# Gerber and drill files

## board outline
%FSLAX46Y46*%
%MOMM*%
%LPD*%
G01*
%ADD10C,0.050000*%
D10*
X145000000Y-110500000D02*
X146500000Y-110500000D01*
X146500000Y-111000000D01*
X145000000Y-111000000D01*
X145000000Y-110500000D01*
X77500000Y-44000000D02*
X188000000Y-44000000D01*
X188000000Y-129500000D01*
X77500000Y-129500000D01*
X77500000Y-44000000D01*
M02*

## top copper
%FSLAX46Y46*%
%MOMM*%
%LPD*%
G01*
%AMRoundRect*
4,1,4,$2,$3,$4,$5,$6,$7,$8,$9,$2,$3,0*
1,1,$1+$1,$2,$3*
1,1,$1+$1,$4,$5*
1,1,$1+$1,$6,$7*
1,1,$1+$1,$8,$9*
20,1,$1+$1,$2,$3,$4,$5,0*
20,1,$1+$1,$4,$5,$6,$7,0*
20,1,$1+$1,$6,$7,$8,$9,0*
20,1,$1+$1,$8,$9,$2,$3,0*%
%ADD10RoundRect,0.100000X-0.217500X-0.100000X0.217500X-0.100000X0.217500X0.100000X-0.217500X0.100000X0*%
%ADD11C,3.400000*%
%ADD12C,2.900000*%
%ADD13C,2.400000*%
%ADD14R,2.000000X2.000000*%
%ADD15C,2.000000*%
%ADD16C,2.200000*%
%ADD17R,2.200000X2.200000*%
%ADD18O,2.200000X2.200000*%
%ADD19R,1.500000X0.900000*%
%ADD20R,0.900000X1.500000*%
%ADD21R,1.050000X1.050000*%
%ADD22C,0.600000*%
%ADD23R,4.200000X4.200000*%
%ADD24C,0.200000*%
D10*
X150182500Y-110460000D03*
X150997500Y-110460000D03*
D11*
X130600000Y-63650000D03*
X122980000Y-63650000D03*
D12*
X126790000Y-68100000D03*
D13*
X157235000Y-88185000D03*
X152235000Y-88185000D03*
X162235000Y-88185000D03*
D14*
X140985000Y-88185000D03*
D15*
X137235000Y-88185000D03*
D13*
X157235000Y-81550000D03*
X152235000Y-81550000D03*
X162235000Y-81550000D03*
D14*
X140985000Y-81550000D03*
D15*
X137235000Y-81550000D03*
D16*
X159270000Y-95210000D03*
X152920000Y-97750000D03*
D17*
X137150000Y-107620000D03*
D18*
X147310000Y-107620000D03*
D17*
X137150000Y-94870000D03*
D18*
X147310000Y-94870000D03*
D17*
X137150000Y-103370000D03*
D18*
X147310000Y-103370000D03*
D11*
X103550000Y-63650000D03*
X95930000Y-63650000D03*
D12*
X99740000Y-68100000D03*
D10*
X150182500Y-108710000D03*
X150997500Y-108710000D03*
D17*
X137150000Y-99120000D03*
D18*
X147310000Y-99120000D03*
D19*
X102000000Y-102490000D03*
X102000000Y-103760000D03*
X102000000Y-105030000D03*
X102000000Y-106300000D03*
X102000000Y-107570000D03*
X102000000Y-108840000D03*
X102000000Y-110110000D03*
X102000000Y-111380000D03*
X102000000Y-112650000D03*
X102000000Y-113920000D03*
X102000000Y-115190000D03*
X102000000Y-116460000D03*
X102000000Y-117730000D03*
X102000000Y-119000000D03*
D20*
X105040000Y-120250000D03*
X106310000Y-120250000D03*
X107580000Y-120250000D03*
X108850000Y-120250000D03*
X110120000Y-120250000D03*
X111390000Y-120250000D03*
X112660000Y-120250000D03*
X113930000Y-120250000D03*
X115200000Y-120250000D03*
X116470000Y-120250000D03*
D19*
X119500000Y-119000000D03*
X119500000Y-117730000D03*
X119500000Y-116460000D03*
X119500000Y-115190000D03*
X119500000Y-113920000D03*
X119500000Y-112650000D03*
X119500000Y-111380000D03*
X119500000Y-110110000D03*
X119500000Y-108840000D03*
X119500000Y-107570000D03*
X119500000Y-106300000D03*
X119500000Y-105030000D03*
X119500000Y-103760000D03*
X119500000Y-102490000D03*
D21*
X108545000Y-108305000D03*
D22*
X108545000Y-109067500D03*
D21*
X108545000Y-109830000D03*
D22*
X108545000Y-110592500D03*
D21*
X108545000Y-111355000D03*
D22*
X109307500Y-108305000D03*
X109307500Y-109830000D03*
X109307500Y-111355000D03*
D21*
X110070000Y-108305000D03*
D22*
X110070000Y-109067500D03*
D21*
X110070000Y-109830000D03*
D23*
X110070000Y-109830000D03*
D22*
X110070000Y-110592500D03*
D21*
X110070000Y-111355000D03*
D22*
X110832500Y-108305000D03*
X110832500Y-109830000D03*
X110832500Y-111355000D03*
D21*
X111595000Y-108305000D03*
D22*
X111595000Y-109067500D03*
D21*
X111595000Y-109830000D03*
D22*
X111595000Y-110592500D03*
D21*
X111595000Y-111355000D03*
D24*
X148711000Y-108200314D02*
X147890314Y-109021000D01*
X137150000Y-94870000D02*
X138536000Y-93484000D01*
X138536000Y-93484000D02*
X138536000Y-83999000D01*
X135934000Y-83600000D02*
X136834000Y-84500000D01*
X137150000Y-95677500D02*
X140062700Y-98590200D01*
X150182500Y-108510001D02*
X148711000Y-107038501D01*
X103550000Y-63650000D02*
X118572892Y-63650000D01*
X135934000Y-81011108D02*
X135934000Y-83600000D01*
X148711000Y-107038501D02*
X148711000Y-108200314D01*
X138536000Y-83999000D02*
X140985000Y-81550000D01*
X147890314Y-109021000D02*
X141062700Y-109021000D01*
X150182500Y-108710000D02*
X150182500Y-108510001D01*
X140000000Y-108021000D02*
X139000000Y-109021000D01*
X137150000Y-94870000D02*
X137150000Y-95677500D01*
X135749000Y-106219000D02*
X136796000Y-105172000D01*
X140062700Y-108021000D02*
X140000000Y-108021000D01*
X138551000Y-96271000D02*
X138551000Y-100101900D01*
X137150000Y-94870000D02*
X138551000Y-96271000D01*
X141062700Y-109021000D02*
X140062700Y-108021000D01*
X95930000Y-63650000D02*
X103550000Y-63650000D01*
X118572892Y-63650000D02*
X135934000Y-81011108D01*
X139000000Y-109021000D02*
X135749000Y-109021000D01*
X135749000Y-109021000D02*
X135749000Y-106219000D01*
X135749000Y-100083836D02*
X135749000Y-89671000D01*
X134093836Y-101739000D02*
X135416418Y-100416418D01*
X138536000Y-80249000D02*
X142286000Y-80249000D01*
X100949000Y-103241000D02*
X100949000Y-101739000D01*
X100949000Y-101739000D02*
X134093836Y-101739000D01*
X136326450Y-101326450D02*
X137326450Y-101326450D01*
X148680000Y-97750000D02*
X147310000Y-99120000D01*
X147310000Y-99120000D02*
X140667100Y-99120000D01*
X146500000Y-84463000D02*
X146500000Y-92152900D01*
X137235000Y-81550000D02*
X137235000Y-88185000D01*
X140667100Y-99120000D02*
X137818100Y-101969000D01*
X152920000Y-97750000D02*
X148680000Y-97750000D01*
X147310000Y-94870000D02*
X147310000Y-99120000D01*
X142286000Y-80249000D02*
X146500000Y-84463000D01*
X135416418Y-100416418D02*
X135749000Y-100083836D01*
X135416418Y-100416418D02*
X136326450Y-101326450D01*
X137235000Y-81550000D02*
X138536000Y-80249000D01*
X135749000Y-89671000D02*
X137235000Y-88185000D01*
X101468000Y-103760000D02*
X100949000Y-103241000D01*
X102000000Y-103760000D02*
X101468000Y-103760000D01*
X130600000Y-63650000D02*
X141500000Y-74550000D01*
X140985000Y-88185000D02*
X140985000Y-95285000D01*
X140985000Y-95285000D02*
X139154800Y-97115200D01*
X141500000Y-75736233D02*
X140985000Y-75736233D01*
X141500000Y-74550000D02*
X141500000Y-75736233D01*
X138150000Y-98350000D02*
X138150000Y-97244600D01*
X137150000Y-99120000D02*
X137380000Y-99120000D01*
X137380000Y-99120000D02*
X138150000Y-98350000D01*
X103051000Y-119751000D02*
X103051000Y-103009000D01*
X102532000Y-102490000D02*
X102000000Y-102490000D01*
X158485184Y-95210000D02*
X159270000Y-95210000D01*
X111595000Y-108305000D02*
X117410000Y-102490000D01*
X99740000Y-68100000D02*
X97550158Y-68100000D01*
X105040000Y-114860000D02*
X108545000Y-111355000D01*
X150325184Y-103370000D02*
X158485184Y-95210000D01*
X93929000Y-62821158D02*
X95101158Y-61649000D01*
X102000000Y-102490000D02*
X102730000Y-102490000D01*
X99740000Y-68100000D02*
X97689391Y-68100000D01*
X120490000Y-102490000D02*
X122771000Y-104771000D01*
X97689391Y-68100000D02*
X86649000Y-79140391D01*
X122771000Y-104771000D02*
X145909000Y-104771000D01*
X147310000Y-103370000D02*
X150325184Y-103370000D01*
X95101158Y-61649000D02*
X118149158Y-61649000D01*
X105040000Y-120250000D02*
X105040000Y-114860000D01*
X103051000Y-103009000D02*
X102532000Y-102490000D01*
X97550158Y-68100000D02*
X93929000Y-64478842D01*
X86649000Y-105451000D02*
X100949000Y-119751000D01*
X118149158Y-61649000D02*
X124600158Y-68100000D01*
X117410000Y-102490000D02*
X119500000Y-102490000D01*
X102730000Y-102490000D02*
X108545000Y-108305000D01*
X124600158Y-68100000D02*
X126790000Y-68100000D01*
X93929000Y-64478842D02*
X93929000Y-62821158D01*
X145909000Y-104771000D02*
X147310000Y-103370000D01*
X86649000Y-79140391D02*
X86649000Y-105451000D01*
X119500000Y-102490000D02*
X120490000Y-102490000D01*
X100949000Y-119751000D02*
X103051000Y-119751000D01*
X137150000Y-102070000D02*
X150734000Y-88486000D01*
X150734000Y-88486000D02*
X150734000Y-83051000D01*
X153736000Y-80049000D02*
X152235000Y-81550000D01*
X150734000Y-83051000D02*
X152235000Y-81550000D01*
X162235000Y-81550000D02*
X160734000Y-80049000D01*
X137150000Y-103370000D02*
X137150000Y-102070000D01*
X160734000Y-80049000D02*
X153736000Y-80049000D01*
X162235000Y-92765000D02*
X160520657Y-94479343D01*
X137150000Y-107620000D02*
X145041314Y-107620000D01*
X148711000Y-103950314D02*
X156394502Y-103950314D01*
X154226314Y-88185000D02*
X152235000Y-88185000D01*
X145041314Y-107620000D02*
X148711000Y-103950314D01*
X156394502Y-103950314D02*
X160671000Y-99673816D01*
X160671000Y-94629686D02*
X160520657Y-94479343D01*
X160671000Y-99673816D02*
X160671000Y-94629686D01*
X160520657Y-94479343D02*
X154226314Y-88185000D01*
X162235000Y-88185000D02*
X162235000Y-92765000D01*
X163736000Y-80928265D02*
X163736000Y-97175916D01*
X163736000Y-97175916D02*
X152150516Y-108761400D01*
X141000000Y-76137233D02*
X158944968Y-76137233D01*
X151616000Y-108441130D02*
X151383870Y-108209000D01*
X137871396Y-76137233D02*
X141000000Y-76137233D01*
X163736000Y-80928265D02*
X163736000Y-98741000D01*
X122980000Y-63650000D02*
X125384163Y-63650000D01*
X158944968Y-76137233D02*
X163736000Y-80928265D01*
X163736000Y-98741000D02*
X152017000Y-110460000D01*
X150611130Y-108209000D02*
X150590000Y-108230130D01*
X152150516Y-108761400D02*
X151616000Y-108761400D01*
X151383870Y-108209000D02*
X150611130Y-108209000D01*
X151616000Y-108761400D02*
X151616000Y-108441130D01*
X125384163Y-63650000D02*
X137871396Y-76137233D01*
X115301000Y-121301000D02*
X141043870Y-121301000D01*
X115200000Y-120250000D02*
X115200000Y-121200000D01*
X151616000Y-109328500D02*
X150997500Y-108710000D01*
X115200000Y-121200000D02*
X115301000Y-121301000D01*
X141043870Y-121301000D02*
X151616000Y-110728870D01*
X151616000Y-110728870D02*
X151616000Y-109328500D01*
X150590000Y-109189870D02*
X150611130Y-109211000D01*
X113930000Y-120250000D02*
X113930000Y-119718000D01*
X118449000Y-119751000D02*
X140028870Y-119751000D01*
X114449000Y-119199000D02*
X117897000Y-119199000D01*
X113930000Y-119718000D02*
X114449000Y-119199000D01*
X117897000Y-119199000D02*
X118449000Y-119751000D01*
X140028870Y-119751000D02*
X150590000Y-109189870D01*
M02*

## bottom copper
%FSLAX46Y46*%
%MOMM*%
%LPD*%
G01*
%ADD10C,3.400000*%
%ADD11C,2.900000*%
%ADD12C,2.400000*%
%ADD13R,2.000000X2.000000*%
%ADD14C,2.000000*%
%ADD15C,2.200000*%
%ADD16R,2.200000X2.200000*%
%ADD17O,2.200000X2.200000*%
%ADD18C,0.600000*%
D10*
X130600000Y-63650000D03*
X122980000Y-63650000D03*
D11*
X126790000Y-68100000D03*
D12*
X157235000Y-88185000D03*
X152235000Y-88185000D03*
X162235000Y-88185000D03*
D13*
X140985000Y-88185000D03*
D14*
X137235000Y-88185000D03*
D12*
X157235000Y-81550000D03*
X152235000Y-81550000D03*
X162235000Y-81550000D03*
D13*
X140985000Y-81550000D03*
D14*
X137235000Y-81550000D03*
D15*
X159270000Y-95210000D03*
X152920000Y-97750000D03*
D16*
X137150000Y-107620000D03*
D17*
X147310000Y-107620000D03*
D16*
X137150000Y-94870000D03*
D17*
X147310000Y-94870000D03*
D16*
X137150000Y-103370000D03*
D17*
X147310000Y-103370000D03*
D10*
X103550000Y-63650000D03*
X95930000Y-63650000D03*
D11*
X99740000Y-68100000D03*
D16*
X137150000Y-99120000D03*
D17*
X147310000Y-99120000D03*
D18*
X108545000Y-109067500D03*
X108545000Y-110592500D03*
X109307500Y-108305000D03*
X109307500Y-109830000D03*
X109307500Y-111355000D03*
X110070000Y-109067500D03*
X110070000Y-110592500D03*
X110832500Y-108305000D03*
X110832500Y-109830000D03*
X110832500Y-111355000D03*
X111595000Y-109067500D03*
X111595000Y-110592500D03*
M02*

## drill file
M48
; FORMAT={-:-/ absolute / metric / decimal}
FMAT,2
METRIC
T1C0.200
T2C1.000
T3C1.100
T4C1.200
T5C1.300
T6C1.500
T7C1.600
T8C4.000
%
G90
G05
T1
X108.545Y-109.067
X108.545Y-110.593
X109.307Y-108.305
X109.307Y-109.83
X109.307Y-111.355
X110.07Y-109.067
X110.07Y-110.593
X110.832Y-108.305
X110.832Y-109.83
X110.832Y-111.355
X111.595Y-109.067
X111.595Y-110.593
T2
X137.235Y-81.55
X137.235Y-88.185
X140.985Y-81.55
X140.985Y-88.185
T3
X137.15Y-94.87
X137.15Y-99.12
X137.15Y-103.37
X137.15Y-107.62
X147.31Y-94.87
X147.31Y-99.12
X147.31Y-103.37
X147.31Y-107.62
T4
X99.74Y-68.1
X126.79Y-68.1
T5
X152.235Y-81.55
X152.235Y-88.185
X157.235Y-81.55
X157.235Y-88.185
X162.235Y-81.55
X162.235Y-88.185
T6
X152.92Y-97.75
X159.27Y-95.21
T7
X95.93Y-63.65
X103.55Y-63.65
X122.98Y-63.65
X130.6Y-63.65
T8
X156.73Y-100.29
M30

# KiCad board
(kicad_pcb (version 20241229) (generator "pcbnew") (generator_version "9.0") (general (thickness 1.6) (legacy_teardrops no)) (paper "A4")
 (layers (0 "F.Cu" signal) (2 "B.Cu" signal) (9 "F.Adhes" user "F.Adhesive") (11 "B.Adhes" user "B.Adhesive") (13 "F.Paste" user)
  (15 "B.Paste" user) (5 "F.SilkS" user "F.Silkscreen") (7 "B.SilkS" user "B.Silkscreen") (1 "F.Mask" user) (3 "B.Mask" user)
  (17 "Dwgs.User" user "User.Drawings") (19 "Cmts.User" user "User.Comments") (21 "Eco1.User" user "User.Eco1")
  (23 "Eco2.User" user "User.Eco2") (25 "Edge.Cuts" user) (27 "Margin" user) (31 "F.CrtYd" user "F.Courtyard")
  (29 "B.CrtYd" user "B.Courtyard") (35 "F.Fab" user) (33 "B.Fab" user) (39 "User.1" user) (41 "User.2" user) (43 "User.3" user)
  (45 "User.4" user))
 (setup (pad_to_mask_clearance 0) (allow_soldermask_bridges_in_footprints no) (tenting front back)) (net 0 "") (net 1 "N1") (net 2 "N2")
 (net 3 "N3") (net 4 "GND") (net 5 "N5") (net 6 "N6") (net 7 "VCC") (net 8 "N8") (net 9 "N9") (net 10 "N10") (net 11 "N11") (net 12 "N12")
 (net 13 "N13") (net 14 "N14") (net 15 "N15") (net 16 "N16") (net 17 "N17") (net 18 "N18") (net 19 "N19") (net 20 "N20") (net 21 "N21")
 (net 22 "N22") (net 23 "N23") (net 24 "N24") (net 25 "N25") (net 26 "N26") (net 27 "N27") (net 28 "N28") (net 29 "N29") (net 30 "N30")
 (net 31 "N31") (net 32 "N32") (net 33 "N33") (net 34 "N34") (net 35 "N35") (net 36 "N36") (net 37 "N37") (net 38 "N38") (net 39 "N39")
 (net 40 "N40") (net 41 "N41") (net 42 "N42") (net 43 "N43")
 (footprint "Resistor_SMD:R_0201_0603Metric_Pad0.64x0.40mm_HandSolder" (layer "F.Cu") (at 150.59 110.46)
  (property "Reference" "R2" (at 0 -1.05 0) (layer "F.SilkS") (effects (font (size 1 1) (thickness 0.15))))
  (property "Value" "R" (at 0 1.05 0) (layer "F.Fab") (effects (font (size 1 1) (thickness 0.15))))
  (pad "" smd roundrect (at -0.4325 0) (size 0.458 0.36) (layers "F.Paste") (roundrect_rratio 0.25))
  (pad "" smd roundrect (at 0.4325 0) (size 0.458 0.36) (layers "F.Paste") (roundrect_rratio 0.25))
  (pad "1" smd roundrect (at -0.4075 0) (size 0.635 0.4) (layers "F.Cu" "F.Mask") (roundrect_rratio 0.25) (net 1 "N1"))
  (pad "2" smd roundrect (at 0.4075 0) (size 0.635 0.4) (layers "F.Cu" "F.Mask") (roundrect_rratio 0.25) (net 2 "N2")))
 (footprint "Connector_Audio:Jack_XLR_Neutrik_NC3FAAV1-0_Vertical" (layer "F.Cu") (at 130.6 63.65)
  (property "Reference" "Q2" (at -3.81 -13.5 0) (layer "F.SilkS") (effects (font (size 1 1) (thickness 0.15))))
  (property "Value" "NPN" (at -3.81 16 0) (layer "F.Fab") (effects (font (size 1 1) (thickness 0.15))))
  (pad "1" thru_hole circle (at 0 0) (size 3.4 3.4) (drill 1.6) (layers "*.Cu" "*.Mask") (remove_unused_layers no) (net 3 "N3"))
  (pad "2" thru_hole circle (at -7.62 0) (size 3.4 3.4) (drill 1.6) (layers "*.Cu" "*.Mask") (remove_unused_layers no) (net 2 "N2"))
  (pad "3" thru_hole circle (at -3.81 4.45) (size 2.9 2.9) (drill 1.2) (layers "*.Cu" "*.Mask") (remove_unused_layers no) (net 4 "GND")))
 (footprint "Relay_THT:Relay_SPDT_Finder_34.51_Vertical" (layer "F.Cu") (at 140.985 88.185)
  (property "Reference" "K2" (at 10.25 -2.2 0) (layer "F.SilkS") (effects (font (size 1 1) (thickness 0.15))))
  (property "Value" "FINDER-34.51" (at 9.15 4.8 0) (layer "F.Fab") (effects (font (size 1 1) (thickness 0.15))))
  (pad "11" thru_hole circle (at 16.25 0) (size 2.4 2.4) (drill 1.3) (layers "*.Cu" "*.Mask") (remove_unused_layers no) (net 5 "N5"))
  (pad "12" thru_hole circle (at 11.25 0) (size 2.4 2.4) (drill 1.3) (layers "*.Cu" "*.Mask") (remove_unused_layers no) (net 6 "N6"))
  (pad "14" thru_hole circle (at 21.25 0) (size 2.4 2.4) (drill 1.3) (layers "*.Cu" "*.Mask") (remove_unused_layers no) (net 6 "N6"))
  (pad "A1" thru_hole rect (at 0 0) (size 2 2) (drill 1) (layers "*.Cu" "*.Mask") (remove_unused_layers no) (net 3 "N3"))
  (pad "A2" thru_hole circle (at -3.75 0) (size 2 2) (drill 1) (layers "*.Cu" "*.Mask") (remove_unused_layers no) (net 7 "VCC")))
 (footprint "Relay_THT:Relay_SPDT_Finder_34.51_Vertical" (layer "F.Cu") (at 140.985 81.55)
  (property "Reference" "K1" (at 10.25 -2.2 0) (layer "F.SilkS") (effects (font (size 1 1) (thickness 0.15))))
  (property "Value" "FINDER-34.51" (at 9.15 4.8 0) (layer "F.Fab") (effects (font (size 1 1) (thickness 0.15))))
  (pad "11" thru_hole circle (at 16.25 0) (size 2.4 2.4) (drill 1.3) (layers "*.Cu" "*.Mask") (remove_unused_layers no) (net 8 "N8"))
  (pad "12" thru_hole circle (at 11.25 0) (size 2.4 2.4) (drill 1.3) (layers "*.Cu" "*.Mask") (remove_unused_layers no) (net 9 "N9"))
  (pad "14" thru_hole circle (at 21.25 0) (size 2.4 2.4) (drill 1.3) (layers "*.Cu" "*.Mask") (remove_unused_layers no) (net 9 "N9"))
  (pad "A1" thru_hole rect (at 0 0) (size 2 2) (drill 1) (layers "*.Cu" "*.Mask") (remove_unused_layers no) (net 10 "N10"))
  (pad "A2" thru_hole circle (at -3.75 0) (size 2 2) (drill 1) (layers "*.Cu" "*.Mask") (remove_unused_layers no) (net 7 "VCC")))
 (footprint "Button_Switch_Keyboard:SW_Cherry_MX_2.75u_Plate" (layer "F.Cu") (at 159.27 95.21)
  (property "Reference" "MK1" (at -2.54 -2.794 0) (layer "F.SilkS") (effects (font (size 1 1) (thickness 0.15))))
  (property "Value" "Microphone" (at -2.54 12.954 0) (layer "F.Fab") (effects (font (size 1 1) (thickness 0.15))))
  (pad "" np_thru_hole circle (at -2.54 5.08) (size 4 4) (drill 4) (layers "*.Cu" "*.Mask"))
  (pad "1" thru_hole circle (at 0 0) (size 2.2 2.2) (drill 1.5) (layers "*.Cu" "*.Mask") (remove_unused_layers no) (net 4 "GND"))
  (pad "2" thru_hole circle (at -6.35 2.54) (size 2.2 2.2) (drill 1.5) (layers "*.Cu" "*.Mask") (remove_unused_layers no) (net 7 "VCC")))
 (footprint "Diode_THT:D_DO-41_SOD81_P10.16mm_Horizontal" (layer "F.Cu") (at 137.15 107.62)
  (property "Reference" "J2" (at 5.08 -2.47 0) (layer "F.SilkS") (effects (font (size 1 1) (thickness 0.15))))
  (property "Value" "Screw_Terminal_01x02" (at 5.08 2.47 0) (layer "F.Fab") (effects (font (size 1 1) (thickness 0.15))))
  (pad "1" thru_hole rect (at 0 0) (size 2.2 2.2) (drill 1.1) (layers "*.Cu" "*.Mask") (remove_unused_layers no) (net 6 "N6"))
  (pad "2" thru_hole oval (at 10.16 0) (size 2.2 2.2) (drill 1.1) (layers "*.Cu" "*.Mask") (remove_unused_layers no) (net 4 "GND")))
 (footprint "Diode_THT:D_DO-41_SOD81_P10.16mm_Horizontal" (layer "F.Cu") (at 137.15 94.87)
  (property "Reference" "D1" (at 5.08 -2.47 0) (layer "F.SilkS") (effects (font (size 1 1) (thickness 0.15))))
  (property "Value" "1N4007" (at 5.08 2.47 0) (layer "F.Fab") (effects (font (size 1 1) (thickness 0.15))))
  (pad "1" thru_hole rect (at 0 0) (size 2.2 2.2) (drill 1.1) (layers "*.Cu" "*.Mask") (remove_unused_layers no) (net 10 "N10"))
  (pad "2" thru_hole oval (at 10.16 0) (size 2.2 2.2) (drill 1.1) (layers "*.Cu" "*.Mask") (remove_unused_layers no) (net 7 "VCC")))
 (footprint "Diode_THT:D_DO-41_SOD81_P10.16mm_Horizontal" (layer "F.Cu") (at 137.15 103.37)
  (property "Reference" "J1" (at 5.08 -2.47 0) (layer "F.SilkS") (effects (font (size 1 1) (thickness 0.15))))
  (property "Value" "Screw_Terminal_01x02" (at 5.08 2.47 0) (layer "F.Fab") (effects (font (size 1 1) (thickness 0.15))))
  (pad "1" thru_hole rect (at 0 0) (size 2.2 2.2) (drill 1.1) (layers "*.Cu" "*.Mask") (remove_unused_layers no) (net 9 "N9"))
  (pad "2" thru_hole oval (at 10.16 0) (size 2.2 2.2) (drill 1.1) (layers "*.Cu" "*.Mask") (remove_unused_layers no) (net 4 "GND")))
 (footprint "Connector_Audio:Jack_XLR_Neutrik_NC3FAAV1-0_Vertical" (layer "F.Cu") (at 103.55 63.65)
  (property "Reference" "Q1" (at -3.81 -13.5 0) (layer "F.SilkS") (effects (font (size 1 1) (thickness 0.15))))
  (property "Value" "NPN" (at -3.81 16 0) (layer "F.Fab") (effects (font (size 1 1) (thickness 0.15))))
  (pad "1" thru_hole circle (at 0 0) (size 3.4 3.4) (drill 1.6) (layers "*.Cu" "*.Mask") (remove_unused_layers no) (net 10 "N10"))
  (pad "2" thru_hole circle (at -7.62 0) (size 3.4 3.4) (drill 1.6) (layers "*.Cu" "*.Mask") (remove_unused_layers no) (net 10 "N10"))
  (pad "3" thru_hole circle (at -3.81 4.45) (size 2.9 2.9) (drill 1.2) (layers "*.Cu" "*.Mask") (remove_unused_layers no) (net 4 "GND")))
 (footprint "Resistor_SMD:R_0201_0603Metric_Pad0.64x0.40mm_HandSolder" (layer "F.Cu") (at 150.59 108.71)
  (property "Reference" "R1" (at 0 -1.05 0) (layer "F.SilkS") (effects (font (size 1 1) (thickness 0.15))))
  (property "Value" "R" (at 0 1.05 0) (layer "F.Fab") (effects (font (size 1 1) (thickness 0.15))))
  (pad "" smd roundrect (at -0.4325 0) (size 0.458 0.36) (layers "F.Paste") (roundrect_rratio 0.25))
  (pad "" smd roundrect (at 0.4325 0) (size 0.458 0.36) (layers "F.Paste") (roundrect_rratio 0.25))
  (pad "1" smd roundrect (at -0.4075 0) (size 0.635 0.4) (layers "F.Cu" "F.Mask") (roundrect_rratio 0.25) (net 10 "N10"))
  (pad "2" smd roundrect (at 0.4075 0) (size 0.635 0.4) (layers "F.Cu" "F.Mask") (roundrect_rratio 0.25) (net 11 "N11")))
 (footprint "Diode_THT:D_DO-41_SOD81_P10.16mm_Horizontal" (layer "F.Cu") (at 137.15 99.12)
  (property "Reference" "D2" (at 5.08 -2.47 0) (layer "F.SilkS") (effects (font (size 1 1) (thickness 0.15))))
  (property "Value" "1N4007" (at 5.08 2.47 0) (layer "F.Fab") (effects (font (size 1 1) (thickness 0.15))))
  (pad "1" thru_hole rect (at 0 0) (size 2.2 2.2) (drill 1.1) (layers "*.Cu" "*.Mask") (remove_unused_layers no) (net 3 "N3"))
  (pad "2" thru_hole oval (at 10.16 0) (size 2.2 2.2) (drill 1.1) (layers "*.Cu" "*.Mask") (remove_unused_layers no) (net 7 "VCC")))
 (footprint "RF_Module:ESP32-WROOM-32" (layer "F.Cu") (at 110.75 110.74)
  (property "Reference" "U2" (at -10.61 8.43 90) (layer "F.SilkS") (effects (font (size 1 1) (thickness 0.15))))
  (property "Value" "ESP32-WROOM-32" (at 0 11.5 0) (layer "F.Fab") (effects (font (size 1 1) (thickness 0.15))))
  (pad "1" smd rect (at -8.75 -8.25) (size 1.5 0.9) (layers "F.Cu" "F.Mask" "F.Paste") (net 4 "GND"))
  (pad "2" smd rect (at -8.75 -6.98) (size 1.5 0.9) (layers "F.Cu" "F.Mask" "F.Paste") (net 7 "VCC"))
  (pad "3" smd rect (at -8.75 -5.71) (size 1.5 0.9) (layers "F.Cu" "F.Mask" "F.Paste") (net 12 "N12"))
  (pad "4" smd rect (at -8.75 -4.44) (size 1.5 0.9) (layers "F.Cu" "F.Mask" "F.Paste") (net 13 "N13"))
  (pad "5" smd rect (at -8.75 -3.17) (size 1.5 0.9) (layers "F.Cu" "F.Mask" "F.Paste") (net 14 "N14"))
  (pad "6" smd rect (at -8.75 -1.9) (size 1.5 0.9) (layers "F.Cu" "F.Mask" "F.Paste") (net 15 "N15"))
  (pad "7" smd rect (at -8.75 -0.63) (size 1.5 0.9) (layers "F.Cu" "F.Mask" "F.Paste") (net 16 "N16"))
  (pad "8" smd rect (at -8.75 0.64) (size 1.5 0.9) (layers "F.Cu" "F.Mask" "F.Paste") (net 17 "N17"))
  (pad "9" smd rect (at -8.75 1.91) (size 1.5 0.9) (layers "F.Cu" "F.Mask" "F.Paste") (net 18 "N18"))
  (pad "10" smd rect (at -8.75 3.18) (size 1.5 0.9) (layers "F.Cu" "F.Mask" "F.Paste") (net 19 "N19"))
  (pad "11" smd rect (at -8.75 4.45) (size 1.5 0.9) (layers "F.Cu" "F.Mask" "F.Paste") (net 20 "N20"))
  (pad "12" smd rect (at -8.75 5.72) (size 1.5 0.9) (layers "F.Cu" "F.Mask" "F.Paste") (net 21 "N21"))
  (pad "13" smd rect (at -8.75 6.99) (size 1.5 0.9) (layers "F.Cu" "F.Mask" "F.Paste") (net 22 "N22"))
  (pad "14" smd rect (at -8.75 8.26) (size 1.5 0.9) (layers "F.Cu" "F.Mask" "F.Paste") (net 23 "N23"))
  (pad "15" smd rect (at -5.71 9.51 90) (size 1.5 0.9) (layers "F.Cu" "F.Mask" "F.Paste") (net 4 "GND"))
  (pad "16" smd rect (at -4.44 9.51 90) (size 1.5 0.9) (layers "F.Cu" "F.Mask" "F.Paste") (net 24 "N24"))
  (pad "17" smd rect (at -3.17 9.51 90) (size 1.5 0.9) (layers "F.Cu" "F.Mask" "F.Paste") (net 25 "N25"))
  (pad "18" smd rect (at -1.9 9.51 90) (size 1.5 0.9) (layers "F.Cu" "F.Mask" "F.Paste") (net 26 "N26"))
  (pad "19" smd rect (at -0.63 9.51 90) (size 1.5 0.9) (layers "F.Cu" "F.Mask" "F.Paste") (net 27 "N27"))
  (pad "20" smd rect (at 0.64 9.51 90) (size 1.5 0.9) (layers "F.Cu" "F.Mask" "F.Paste") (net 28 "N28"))
  (pad "21" smd rect (at 1.91 9.51 90) (size 1.5 0.9) (layers "F.Cu" "F.Mask" "F.Paste") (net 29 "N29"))
  (pad "22" smd rect (at 3.18 9.51 90) (size 1.5 0.9) (layers "F.Cu" "F.Mask" "F.Paste") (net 1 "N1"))
  (pad "23" smd rect (at 4.45 9.51 90) (size 1.5 0.9) (layers "F.Cu" "F.Mask" "F.Paste") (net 11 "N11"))
  (pad "24" smd rect (at 5.72 9.51 90) (size 1.5 0.9) (layers "F.Cu" "F.Mask" "F.Paste") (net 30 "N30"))
  (pad "25" smd rect (at 8.75 8.26) (size 1.5 0.9) (layers "F.Cu" "F.Mask" "F.Paste") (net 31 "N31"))
  (pad "26" smd rect (at 8.75 6.99) (size 1.5 0.9) (layers "F.Cu" "F.Mask" "F.Paste") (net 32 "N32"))
  (pad "27" smd rect (at 8.75 5.72) (size 1.5 0.9) (layers "F.Cu" "F.Mask" "F.Paste") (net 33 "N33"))
  (pad "28" smd rect (at 8.75 4.45) (size 1.5 0.9) (layers "F.Cu" "F.Mask" "F.Paste") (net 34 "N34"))
  (pad "29" smd rect (at 8.75 3.18) (size 1.5 0.9) (layers "F.Cu" "F.Mask" "F.Paste") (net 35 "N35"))
  (pad "30" smd rect (at 8.75 1.91) (size 1.5 0.9) (layers "F.Cu" "F.Mask" "F.Paste") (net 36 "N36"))
  (pad "31" smd rect (at 8.75 0.64) (size 1.5 0.9) (layers "F.Cu" "F.Mask" "F.Paste") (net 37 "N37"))
  (pad "32" smd rect (at 8.75 -0.63) (size 1.5 0.9) (layers "F.Cu" "F.Mask" "F.Paste") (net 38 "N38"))
  (pad "33" smd rect (at 8.75 -1.9) (size 1.5 0.9) (layers "F.Cu" "F.Mask" "F.Paste") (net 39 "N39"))
  (pad "34" smd rect (at 8.75 -3.17) (size 1.5 0.9) (layers "F.Cu" "F.Mask" "F.Paste") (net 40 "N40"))
  (pad "35" smd rect (at 8.75 -4.44) (size 1.5 0.9) (layers "F.Cu" "F.Mask" "F.Paste") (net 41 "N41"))
  (pad "36" smd rect (at 8.75 -5.71) (size 1.5 0.9) (layers "F.Cu" "F.Mask" "F.Paste") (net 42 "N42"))
  (pad "37" smd rect (at 8.75 -6.98) (size 1.5 0.9) (layers "F.Cu" "F.Mask" "F.Paste") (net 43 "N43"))
  (pad "38" smd rect (at 8.75 -8.25) (size 1.5 0.9) (layers "F.Cu" "F.Mask" "F.Paste") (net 4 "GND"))
  (pad "39" smd rect (at -2.205 -2.435) (size 1.05 1.05) (layers "F.Cu" "F.Paste") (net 4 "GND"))
  (pad "39" thru_hole circle (at -2.205 -1.6725) (size 0.6 0.6) (drill 0.2) (layers "*.Cu" "F.Mask") (remove_unused_layers no) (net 4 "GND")
   (zone_connect 2))
  (pad "39" smd rect (at -2.205 -0.91) (size 1.05 1.05) (layers "F.Cu" "F.Paste") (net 4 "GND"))
  (pad "39" thru_hole circle (at -2.205 -0.1475) (size 0.6 0.6) (drill 0.2) (layers "*.Cu" "F.Mask") (remove_unused_layers no) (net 4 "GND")
   (zone_connect 2))
  (pad "39" smd rect (at -2.205 0.615) (size 1.05 1.05) (layers "F.Cu" "F.Paste") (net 4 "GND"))
  (pad "39" thru_hole circle (at -1.4425 -2.435) (size 0.6 0.6) (drill 0.2) (layers "*.Cu" "F.Mask") (remove_unused_layers no) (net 4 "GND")
   (zone_connect 2))
  (pad "39" thru_hole circle (at -1.4425 -0.91) (size 0.6 0.6) (drill 0.2) (layers "*.Cu" "F.Mask") (remove_unused_layers no) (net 4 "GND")
   (zone_connect 2))
  (pad "39" thru_hole circle (at -1.4425 0.615) (size 0.6 0.6) (drill 0.2) (layers "*.Cu" "F.Mask") (remove_unused_layers no) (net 4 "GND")
   (zone_connect 2))
  (pad "39" smd rect (at -0.68 -2.435) (size 1.05 1.05) (layers "F.Cu" "F.Paste") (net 4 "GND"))
  (pad "39" thru_hole circle (at -0.68 -1.6725) (size 0.6 0.6) (drill 0.2) (layers "*.Cu" "F.Mask") (remove_unused_layers no) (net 4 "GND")
   (zone_connect 2))
  (pad "39" smd rect (at -0.68 -0.91) (size 1.05 1.05) (layers "F.Cu" "F.Paste") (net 4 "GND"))
  (pad "39" smd rect (at -0.68 -0.91) (size 4.2 4.2) (layers "F.Cu" "F.Mask") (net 4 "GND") (zone_connect 2))
  (pad "39" thru_hole circle (at -0.68 -0.1475) (size 0.6 0.6) (drill 0.2) (layers "*.Cu" "F.Mask") (remove_unused_layers no) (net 4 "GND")
   (zone_connect 2))
  (pad "39" smd rect (at -0.68 0.615) (size 1.05 1.05) (layers "F.Cu" "F.Paste") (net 4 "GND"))
  (pad "39" thru_hole circle (at 0.0825 -2.435) (size 0.6 0.6) (drill 0.2) (layers "*.Cu" "F.Mask") (remove_unused_layers no) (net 4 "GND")
   (zone_connect 2))
  (pad "39" thru_hole circle (at 0.0825 -0.91) (size 0.6 0.6) (drill 0.2) (layers "*.Cu" "F.Mask") (remove_unused_layers no) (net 4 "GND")
   (zone_connect 2))
  (pad "39" thru_hole circle (at 0.0825 0.615) (size 0.6 0.6) (drill 0.2) (layers "*.Cu" "F.Mask") (remove_unused_layers no) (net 4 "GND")
   (zone_connect 2))
  (pad "39" smd rect (at 0.845 -2.435) (size 1.05 1.05) (layers "F.Cu" "F.Paste") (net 4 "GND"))
  (pad "39" thru_hole circle (at 0.845 -1.6725) (size 0.6 0.6) (drill 0.2) (layers "*.Cu" "F.Mask") (remove_unused_layers no) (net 4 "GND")
   (zone_connect 2))
  (pad "39" smd rect (at 0.845 -0.91) (size 1.05 1.05) (layers "F.Cu" "F.Paste") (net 4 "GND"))
  (pad "39" thru_hole circle (at 0.845 -0.1475) (size 0.6 0.6) (drill 0.2) (layers "*.Cu" "F.Mask") (remove_unused_layers no) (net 4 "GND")
   (zone_connect 2))
  (pad "39" smd rect (at 0.845 0.615) (size 1.05 1.05) (layers "F.Cu" "F.Paste") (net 4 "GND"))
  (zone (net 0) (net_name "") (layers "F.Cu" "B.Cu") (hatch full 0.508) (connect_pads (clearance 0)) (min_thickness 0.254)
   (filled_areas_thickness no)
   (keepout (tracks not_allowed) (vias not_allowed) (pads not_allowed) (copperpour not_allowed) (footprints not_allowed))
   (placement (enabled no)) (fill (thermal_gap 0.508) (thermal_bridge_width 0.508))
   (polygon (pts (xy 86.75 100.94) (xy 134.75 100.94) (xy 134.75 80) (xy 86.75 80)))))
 (gr_rect (start 145 110.5) (end 146.5 111) (stroke (width 0.05) (type default)) (fill no) (layer "Edge.Cuts"))
 (gr_rect (start 77.5 44) (end 188 129.5) (stroke (width 0.05) (type default)) (fill no) (layer "Edge.Cuts"))
 (segment (start 148.711 108.200314) (end 147.890314 109.021) (width 0.2) (layer "F.Cu") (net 10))
 (segment (start 137.15 94.87) (end 138.536 93.484) (width 0.2) (layer "F.Cu") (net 10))
 (segment (start 138.536 93.484) (end 138.536 83.999) (width 0.2) (layer "F.Cu") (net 10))
 (segment (start 135.934 83.6) (end 136.834 84.5) (width 0.2) (layer "F.Cu") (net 10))
 (segment (start 137.15 95.6775) (end 140.0627 98.5902) (width 0.2) (layer "F.Cu") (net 10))
 (segment (start 150.1825 108.510001) (end 148.711 107.038501) (width 0.2) (layer "F.Cu") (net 10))
 (segment (start 103.55 63.65) (end 118.572892 63.65) (width 0.2) (layer "F.Cu") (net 10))
 (segment (start 135.934 81.011108) (end 135.934 83.6) (width 0.2) (layer "F.Cu") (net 10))
 (segment (start 148.711 107.038501) (end 148.711 108.200314) (width 0.2) (layer "F.Cu") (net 10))
 (segment (start 138.536 83.999) (end 140.985 81.55) (width 0.2) (layer "F.Cu") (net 10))
 (segment (start 147.890314 109.021) (end 141.0627 109.021) (width 0.2) (layer "F.Cu") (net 10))
 (segment (start 150.1825 108.71) (end 150.1825 108.510001) (width 0.2) (layer "F.Cu") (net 10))
 (segment (start 140 108.021) (end 139 109.021) (width 0.2) (layer "F.Cu") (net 10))
 (segment (start 137.15 94.87) (end 137.15 95.6775) (width 0.2) (layer "F.Cu") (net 10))
 (segment (start 135.749 106.219) (end 136.796 105.172) (width 0.2) (layer "F.Cu") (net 10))
 (segment (start 140.0627 108.021) (end 140 108.021) (width 0.2) (layer "F.Cu") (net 10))
 (segment (start 138.551 96.271) (end 138.551 100.1019) (width 0.2) (layer "F.Cu") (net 10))
 (segment (start 137.15 94.87) (end 138.551 96.271) (width 0.2) (layer "F.Cu") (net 10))
 (segment (start 141.0627 109.021) (end 140.0627 108.021) (width 0.2) (layer "F.Cu") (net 10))
 (segment (start 95.93 63.65) (end 103.55 63.65) (width 0.2) (layer "F.Cu") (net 10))
 (segment (start 118.572892 63.65) (end 135.934 81.011108) (width 0.2) (layer "F.Cu") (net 10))
 (segment (start 139 109.021) (end 135.749 109.021) (width 0.2) (layer "F.Cu") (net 10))
 (segment (start 135.749 109.021) (end 135.749 106.219) (width 0.2) (layer "F.Cu") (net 10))
 (segment (start 135.749 100.083836) (end 135.749 89.671) (width 0.2) (layer "F.Cu") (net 7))
 (segment (start 134.093836 101.739) (end 135.416418 100.416418) (width 0.2) (layer "F.Cu") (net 7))
 (segment (start 138.536 80.249) (end 142.286 80.249) (width 0.2) (layer "F.Cu") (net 7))
 (segment (start 100.949 103.241) (end 100.949 101.739) (width 0.2) (layer "F.Cu") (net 7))
 (segment (start 100.949 101.739) (end 134.093836 101.739) (width 0.2) (layer "F.Cu") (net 7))
 (segment (start 136.32645 101.32645) (end 137.32645 101.32645) (width 0.2) (layer "F.Cu") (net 7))
 (segment (start 148.68 97.75) (end 147.31 99.12) (width 0.2) (layer "F.Cu") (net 7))
 (segment (start 147.31 99.12) (end 140.6671 99.12) (width 0.2) (layer "F.Cu") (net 7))
 (segment (start 146.5 84.463) (end 146.5 92.1529) (width 0.2) (layer "F.Cu") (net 7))
 (segment (start 137.235 81.55) (end 137.235 88.185) (width 0.2) (layer "F.Cu") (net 7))
 (segment (start 140.6671 99.12) (end 137.8181 101.969) (width 0.2) (layer "F.Cu") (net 7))
 (segment (start 152.92 97.75) (end 148.68 97.75) (width 0.2) (layer "F.Cu") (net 7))
 (segment (start 147.31 94.87) (end 147.31 99.12) (width 0.2) (layer "F.Cu") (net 7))
 (segment (start 142.286 80.249) (end 146.5 84.463) (width 0.2) (layer "F.Cu") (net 7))
 (segment (start 135.416418 100.416418) (end 135.749 100.083836) (width 0.2) (layer "F.Cu") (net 7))
 (segment (start 135.416418 100.416418) (end 136.32645 101.32645) (width 0.2) (layer "F.Cu") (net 7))
 (segment (start 137.235 81.55) (end 138.536 80.249) (width 0.2) (layer "F.Cu") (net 7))
 (segment (start 135.749 89.671) (end 137.235 88.185) (width 0.2) (layer "F.Cu") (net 7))
 (segment (start 101.468 103.76) (end 100.949 103.241) (width 0.2) (layer "F.Cu") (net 7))
 (segment (start 102 103.76) (end 101.468 103.76) (width 0.2) (layer "F.Cu") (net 7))
 (segment (start 130.6 63.65) (end 141.5 74.55) (width 0.2) (layer "F.Cu") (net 3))
 (segment (start 140.985 88.185) (end 140.985 95.285) (width 0.2) (layer "F.Cu") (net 3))
 (segment (start 140.985 95.285) (end 139.1548 97.1152) (width 0.2) (layer "F.Cu") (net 3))
 (segment (start 141.5 75.736233) (end 140.985 75.736233) (width 0.2) (layer "F.Cu") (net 3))
 (segment (start 141.5 74.55) (end 141.5 75.736233) (width 0.2) (layer "F.Cu") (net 3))
 (segment (start 138.15 98.35) (end 138.15 97.2446) (width 0.2) (layer "F.Cu") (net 3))
 (segment (start 137.15 99.12) (end 137.38 99.12) (width 0.2) (layer "F.Cu") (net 3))
 (segment (start 137.38 99.12) (end 138.15 98.35) (width 0.2) (layer "F.Cu") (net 3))
 (segment (start 103.051 119.751) (end 103.051 103.009) (width 0.2) (layer "F.Cu") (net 4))
 (segment (start 102.532 102.49) (end 102 102.49) (width 0.2) (layer "F.Cu") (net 4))
 (segment (start 158.485184 95.21) (end 159.27 95.21) (width 0.2) (layer "F.Cu") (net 4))
 (segment (start 111.595 108.305) (end 117.41 102.49) (width 0.2) (layer "F.Cu") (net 4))
 (segment (start 99.74 68.1) (end 97.550158 68.1) (width 0.2) (layer "F.Cu") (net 4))
 (segment (start 105.04 114.86) (end 108.545 111.355) (width 0.2) (layer "F.Cu") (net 4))
 (segment (start 150.325184 103.37) (end 158.485184 95.21) (width 0.2) (layer "F.Cu") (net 4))
 (segment (start 93.929 62.821158) (end 95.101158 61.649) (width 0.2) (layer "F.Cu") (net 4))
 (segment (start 102 102.49) (end 102.73 102.49) (width 0.2) (layer "F.Cu") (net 4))
 (segment (start 99.74 68.1) (end 97.689391 68.1) (width 0.2) (layer "F.Cu") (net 4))
 (segment (start 120.49 102.49) (end 122.771 104.771) (width 0.2) (layer "F.Cu") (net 4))
 (segment (start 97.689391 68.1) (end 86.649 79.140391) (width 0.2) (layer "F.Cu") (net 4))
 (segment (start 122.771 104.771) (end 145.909 104.771) (width 0.2) (layer "F.Cu") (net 4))
 (segment (start 147.31 103.37) (end 150.325184 103.37) (width 0.2) (layer "F.Cu") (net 4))
 (segment (start 95.101158 61.649) (end 118.149158 61.649) (width 0.2) (layer "F.Cu") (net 4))
 (segment (start 105.04 120.25) (end 105.04 114.86) (width 0.2) (layer "F.Cu") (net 4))
 (segment (start 103.051 103.009) (end 102.532 102.49) (width 0.2) (layer "F.Cu") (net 4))
 (segment (start 97.550158 68.1) (end 93.929 64.478842) (width 0.2) (layer "F.Cu") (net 4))
 (segment (start 86.649 105.451) (end 100.949 119.751) (width 0.2) (layer "F.Cu") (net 4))
 (segment (start 118.149158 61.649) (end 124.600158 68.1) (width 0.2) (layer "F.Cu") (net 4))
 (segment (start 117.41 102.49) (end 119.5 102.49) (width 0.2) (layer "F.Cu") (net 4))
 (segment (start 102.73 102.49) (end 108.545 108.305) (width 0.2) (layer "F.Cu") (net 4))
 (segment (start 124.600158 68.1) (end 126.79 68.1) (width 0.2) (layer "F.Cu") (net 4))
 (segment (start 93.929 64.478842) (end 93.929 62.821158) (width 0.2) (layer "F.Cu") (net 4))
 (segment (start 145.909 104.771) (end 147.31 103.37) (width 0.2) (layer "F.Cu") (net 4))
 (segment (start 86.649 79.140391) (end 86.649 105.451) (width 0.2) (layer "F.Cu") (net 4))
 (segment (start 119.5 102.49) (end 120.49 102.49) (width 0.2) (layer "F.Cu") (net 4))
 (segment (start 100.949 119.751) (end 103.051 119.751) (width 0.2) (layer "F.Cu") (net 4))
 (segment (start 137.15 102.07) (end 150.734 88.486) (width 0.2) (layer "F.Cu") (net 9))
 (segment (start 150.734 88.486) (end 150.734 83.051) (width 0.2) (layer "F.Cu") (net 9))
 (segment (start 153.736 80.049) (end 152.235 81.55) (width 0.2) (layer "F.Cu") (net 9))
 (segment (start 150.734 83.051) (end 152.235 81.55) (width 0.2) (layer "F.Cu") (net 9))
 (segment (start 162.235 81.55) (end 160.734 80.049) (width 0.2) (layer "F.Cu") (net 9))
 (segment (start 137.15 103.37) (end 137.15 102.07) (width 0.2) (layer "F.Cu") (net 9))
 (segment (start 160.734 80.049) (end 153.736 80.049) (width 0.2) (layer "F.Cu") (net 9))
 (segment (start 162.235 92.765) (end 160.520657 94.479343) (width 0.2) (layer "F.Cu") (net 6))
 (segment (start 137.15 107.62) (end 145.041314 107.62) (width 0.2) (layer "F.Cu") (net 6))
 (segment (start 148.711 103.950314) (end 156.394502 103.950314) (width 0.2) (layer "F.Cu") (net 6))
 (segment (start 154.226314 88.185) (end 152.235 88.185) (width 0.2) (layer "F.Cu") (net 6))
 (segment (start 145.041314 107.62) (end 148.711 103.950314) (width 0.2) (layer "F.Cu") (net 6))
 (segment (start 156.394502 103.950314) (end 160.671 99.673816) (width 0.2) (layer "F.Cu") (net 6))
 (segment (start 160.671 94.629686) (end 160.520657 94.479343) (width 0.2) (layer "F.Cu") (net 6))
 (segment (start 160.671 99.673816) (end 160.671 94.629686) (width 0.2) (layer "F.Cu") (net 6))
 (segment (start 160.520657 94.479343) (end 154.226314 88.185) (width 0.2) (layer "F.Cu") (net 6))
 (segment (start 162.235 88.185) (end 162.235 92.765) (width 0.2) (layer "F.Cu") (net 6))
 (segment (start 163.736 80.928265) (end 163.736 97.175916) (width 0.2) (layer "F.Cu") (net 2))
 (segment (start 163.736 97.175916) (end 152.150516 108.7614) (width 0.2) (layer "F.Cu") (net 2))
 (segment (start 141 76.137233) (end 158.944968 76.137233) (width 0.2) (layer "F.Cu") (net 2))
 (segment (start 151.616 108.44113) (end 151.38387 108.209) (width 0.2) (layer "F.Cu") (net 2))
 (segment (start 137.871396 76.137233) (end 141 76.137233) (width 0.2) (layer "F.Cu") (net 2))
 (segment (start 163.736 80.928265) (end 163.736 98.741) (width 0.2) (layer "F.Cu") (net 2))
 (segment (start 122.98 63.65) (end 125.384163 63.65) (width 0.2) (layer "F.Cu") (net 2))
 (segment (start 158.944968 76.137233) (end 163.736 80.928265) (width 0.2) (layer "F.Cu") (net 2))
 (segment (start 163.736 98.741) (end 152.017 110.46) (width 0.2) (layer "F.Cu") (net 2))
 (segment (start 150.61113 108.209) (end 150.59 108.23013) (width 0.2) (layer "F.Cu") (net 2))
 (segment (start 152.150516 108.7614) (end 151.616 108.7614) (width 0.2) (layer "F.Cu") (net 2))
 (segment (start 151.38387 108.209) (end 150.61113 108.209) (width 0.2) (layer "F.Cu") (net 2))
 (segment (start 151.616 108.7614) (end 151.616 108.44113) (width 0.2) (layer "F.Cu") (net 2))
 (segment (start 125.384163 63.65) (end 137.871396 76.137233) (width 0.2) (layer "F.Cu") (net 2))
 (segment (start 115.301 121.301) (end 141.04387 121.301) (width 0.2) (layer "F.Cu") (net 11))
 (segment (start 115.2 120.25) (end 115.2 121.2) (width 0.2) (layer "F.Cu") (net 11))
 (segment (start 151.616 109.3285) (end 150.9975 108.71) (width 0.2) (layer "F.Cu") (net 11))
 (segment (start 115.2 121.2) (end 115.301 121.301) (width 0.2) (layer "F.Cu") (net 11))
 (segment (start 141.04387 121.301) (end 151.616 110.72887) (width 0.2) (layer "F.Cu") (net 11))
 (segment (start 151.616 110.72887) (end 151.616 109.3285) (width 0.2) (layer "F.Cu") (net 11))
 (segment (start 150.59 109.18987) (end 150.61113 109.211) (width 0.2) (layer "F.Cu") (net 1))
 (segment (start 113.93 120.25) (end 113.93 119.718) (width 0.2) (layer "F.Cu") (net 1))
 (segment (start 118.449 119.751) (end 140.02887 119.751) (width 0.2) (layer "F.Cu") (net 1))
 (segment (start 114.449 119.199) (end 117.897 119.199) (width 0.2) (layer "F.Cu") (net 1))
 (segment (start 113.93 119.718) (end 114.449 119.199) (width 0.2) (layer "F.Cu") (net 1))
 (segment (start 117.897 119.199) (end 118.449 119.751) (width 0.2) (layer "F.Cu") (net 1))
 (segment (start 140.02887 119.751) (end 150.59 109.18987) (width 0.2) (layer "F.Cu") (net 1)))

